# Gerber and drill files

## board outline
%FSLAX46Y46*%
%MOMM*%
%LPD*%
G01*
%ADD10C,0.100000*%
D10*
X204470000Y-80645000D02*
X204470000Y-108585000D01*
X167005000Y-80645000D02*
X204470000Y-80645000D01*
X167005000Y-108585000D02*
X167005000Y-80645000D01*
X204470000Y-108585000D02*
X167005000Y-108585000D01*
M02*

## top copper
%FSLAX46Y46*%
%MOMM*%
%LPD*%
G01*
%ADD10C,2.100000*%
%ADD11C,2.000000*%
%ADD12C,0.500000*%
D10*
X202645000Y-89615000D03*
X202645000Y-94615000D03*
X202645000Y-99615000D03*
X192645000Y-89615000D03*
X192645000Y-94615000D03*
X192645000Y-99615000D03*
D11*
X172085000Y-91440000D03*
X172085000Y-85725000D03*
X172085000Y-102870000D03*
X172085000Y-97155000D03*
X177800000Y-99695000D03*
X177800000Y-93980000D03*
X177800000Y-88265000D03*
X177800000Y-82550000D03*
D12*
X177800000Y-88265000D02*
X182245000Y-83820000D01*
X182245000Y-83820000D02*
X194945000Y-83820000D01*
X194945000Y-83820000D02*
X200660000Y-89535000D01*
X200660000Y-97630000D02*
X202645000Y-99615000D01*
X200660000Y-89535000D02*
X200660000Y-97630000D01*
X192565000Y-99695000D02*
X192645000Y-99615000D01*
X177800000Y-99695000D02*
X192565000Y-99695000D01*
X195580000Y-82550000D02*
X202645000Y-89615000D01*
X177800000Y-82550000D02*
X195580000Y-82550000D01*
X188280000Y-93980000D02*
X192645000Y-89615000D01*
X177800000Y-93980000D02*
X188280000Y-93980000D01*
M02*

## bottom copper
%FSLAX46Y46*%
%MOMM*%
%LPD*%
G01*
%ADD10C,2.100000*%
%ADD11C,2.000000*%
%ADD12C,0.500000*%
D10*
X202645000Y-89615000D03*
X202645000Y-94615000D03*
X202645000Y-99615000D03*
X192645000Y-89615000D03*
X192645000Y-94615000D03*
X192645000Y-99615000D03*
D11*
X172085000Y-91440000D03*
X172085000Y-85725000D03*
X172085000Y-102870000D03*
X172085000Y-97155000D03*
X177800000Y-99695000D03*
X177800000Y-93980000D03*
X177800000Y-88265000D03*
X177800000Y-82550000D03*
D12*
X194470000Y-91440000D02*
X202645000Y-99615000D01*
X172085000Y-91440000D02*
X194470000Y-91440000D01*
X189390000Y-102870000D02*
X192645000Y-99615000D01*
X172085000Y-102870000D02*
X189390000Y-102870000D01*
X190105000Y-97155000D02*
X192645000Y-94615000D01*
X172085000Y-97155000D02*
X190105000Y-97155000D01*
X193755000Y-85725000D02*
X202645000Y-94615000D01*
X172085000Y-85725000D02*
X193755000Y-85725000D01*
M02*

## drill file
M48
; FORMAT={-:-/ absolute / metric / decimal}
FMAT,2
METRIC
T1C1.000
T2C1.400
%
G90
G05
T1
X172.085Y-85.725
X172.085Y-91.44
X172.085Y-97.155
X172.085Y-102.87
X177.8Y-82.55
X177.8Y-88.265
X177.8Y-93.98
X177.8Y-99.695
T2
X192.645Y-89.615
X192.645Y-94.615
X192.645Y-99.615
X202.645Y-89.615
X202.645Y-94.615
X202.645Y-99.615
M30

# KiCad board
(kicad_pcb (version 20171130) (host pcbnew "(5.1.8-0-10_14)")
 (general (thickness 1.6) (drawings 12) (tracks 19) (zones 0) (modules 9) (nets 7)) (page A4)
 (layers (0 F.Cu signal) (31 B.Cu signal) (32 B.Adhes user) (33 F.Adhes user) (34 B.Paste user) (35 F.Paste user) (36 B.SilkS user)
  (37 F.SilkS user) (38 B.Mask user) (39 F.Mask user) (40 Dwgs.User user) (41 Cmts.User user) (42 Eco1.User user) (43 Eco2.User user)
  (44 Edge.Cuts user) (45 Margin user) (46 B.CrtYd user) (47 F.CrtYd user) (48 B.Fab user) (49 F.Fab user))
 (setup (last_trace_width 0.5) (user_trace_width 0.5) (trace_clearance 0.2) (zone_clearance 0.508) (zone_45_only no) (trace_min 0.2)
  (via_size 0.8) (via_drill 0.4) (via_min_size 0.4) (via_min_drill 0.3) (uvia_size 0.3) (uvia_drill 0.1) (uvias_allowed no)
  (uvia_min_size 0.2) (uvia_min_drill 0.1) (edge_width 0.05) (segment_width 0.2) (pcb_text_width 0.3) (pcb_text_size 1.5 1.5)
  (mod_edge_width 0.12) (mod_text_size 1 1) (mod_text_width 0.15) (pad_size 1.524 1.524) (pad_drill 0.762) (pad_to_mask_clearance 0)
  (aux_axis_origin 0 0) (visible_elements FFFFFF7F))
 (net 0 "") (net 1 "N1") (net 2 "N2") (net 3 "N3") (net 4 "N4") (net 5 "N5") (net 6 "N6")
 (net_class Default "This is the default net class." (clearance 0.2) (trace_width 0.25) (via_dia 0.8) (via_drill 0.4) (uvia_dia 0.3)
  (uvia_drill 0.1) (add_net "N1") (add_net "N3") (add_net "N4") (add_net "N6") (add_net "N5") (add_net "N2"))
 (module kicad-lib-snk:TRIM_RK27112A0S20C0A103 (layer F.Cu) (at 207.645 94.615)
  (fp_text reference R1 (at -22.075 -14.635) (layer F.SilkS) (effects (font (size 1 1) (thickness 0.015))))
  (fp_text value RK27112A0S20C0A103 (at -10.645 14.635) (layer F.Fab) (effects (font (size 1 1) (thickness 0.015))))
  (pad 3_1 thru_hole circle (at -5 -5) (size 2.1 2.1) (drill 1.4) (layers *.Cu *.Mask) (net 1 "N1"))
  (pad 2_1 thru_hole circle (at -5 0) (size 2.1 2.1) (drill 1.4) (layers *.Cu *.Mask) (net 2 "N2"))
  (pad 1_1 thru_hole circle (at -5 5) (size 2.1 2.1) (drill 1.4) (layers *.Cu *.Mask) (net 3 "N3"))
  (pad 3_2 thru_hole circle (at -15 -5) (size 2.1 2.1) (drill 1.4) (layers *.Cu *.Mask) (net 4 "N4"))
  (pad 2_2 thru_hole circle (at -15 0) (size 2.1 2.1) (drill 1.4) (layers *.Cu *.Mask) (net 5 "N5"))
  (pad 1_2 thru_hole circle (at -15 5) (size 2.1 2.1) (drill 1.4) (layers *.Cu *.Mask) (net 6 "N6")))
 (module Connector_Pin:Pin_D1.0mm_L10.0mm (layer F.Cu) (at 172.085 91.44)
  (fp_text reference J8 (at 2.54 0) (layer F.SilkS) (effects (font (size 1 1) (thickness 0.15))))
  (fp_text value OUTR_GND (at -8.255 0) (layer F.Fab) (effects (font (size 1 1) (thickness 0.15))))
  (pad 1 thru_hole circle (at 0 0) (size 2 2) (drill 1) (layers *.Cu *.Mask) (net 3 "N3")))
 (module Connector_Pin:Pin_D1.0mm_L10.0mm (layer F.Cu) (at 172.085 85.725)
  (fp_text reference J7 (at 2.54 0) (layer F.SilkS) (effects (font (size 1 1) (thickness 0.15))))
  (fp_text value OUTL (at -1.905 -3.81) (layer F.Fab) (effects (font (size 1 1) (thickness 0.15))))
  (pad 1 thru_hole circle (at 0 0) (size 2 2) (drill 1) (layers *.Cu *.Mask) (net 2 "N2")))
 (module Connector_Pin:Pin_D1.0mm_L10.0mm (layer F.Cu) (at 172.085 102.87)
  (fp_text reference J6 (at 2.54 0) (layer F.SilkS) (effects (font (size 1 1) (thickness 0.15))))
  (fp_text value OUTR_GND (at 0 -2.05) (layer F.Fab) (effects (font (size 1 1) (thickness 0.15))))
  (pad 1 thru_hole circle (at 0 0) (size 2 2) (drill 1) (layers *.Cu *.Mask) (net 6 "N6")))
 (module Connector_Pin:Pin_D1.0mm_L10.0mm (layer F.Cu) (at 172.085 97.155)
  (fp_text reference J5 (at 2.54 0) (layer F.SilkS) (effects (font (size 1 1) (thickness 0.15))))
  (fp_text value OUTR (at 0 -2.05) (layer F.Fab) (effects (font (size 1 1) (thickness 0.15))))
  (pad 1 thru_hole circle (at 0 0) (size 2 2) (drill 1) (layers *.Cu *.Mask) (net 5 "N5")))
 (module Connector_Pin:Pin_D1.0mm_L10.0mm (layer F.Cu) (at 177.8 99.695)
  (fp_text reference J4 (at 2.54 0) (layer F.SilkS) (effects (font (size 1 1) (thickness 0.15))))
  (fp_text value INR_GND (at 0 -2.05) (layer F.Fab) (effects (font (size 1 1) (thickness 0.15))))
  (pad 1 thru_hole circle (at 0 0) (size 2 2) (drill 1) (layers *.Cu *.Mask) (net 6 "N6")))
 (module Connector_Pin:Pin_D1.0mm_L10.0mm (layer F.Cu) (at 177.8 93.98)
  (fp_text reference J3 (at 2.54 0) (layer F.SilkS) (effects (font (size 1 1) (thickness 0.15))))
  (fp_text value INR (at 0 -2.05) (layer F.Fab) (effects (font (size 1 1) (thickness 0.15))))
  (pad 1 thru_hole circle (at 0 0) (size 2 2) (drill 1) (layers *.Cu *.Mask) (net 4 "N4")))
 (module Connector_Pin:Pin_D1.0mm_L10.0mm (layer F.Cu) (at 177.8 88.265)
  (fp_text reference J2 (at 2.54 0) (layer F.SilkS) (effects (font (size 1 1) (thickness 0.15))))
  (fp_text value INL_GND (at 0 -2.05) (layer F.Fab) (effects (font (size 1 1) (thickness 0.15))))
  (pad 1 thru_hole circle (at 0 0) (size 2 2) (drill 1) (layers *.Cu *.Mask) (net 3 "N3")))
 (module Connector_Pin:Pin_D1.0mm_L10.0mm (layer F.Cu) (at 177.8 82.55)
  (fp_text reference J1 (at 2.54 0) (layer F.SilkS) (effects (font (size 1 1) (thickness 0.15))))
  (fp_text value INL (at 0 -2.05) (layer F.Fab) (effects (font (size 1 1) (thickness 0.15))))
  (pad 1 thru_hole circle (at 0 0) (size 2 2) (drill 1) (layers *.Cu *.Mask) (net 1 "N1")))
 (gr_line (start 204.47 80.645) (end 204.47 108.585) (layer Edge.Cuts) (width 0.1))
 (gr_line (start 167.005 80.645) (end 204.47 80.645) (layer Edge.Cuts) (width 0.1))
 (gr_line (start 167.005 108.585) (end 167.005 80.645) (layer Edge.Cuts) (width 0.1))
 (gr_line (start 204.47 108.585) (end 167.005 108.585) (layer Edge.Cuts) (width 0.1))
 (segment (start 177.8 88.265) (end 182.245 83.82) (width 0.5) (layer F.Cu) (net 3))
 (segment (start 182.245 83.82) (end 194.945 83.82) (width 0.5) (layer F.Cu) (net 3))
 (segment (start 194.945 83.82) (end 200.66 89.535) (width 0.5) (layer F.Cu) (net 3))
 (segment (start 200.66 97.63) (end 202.645 99.615) (width 0.5) (layer F.Cu) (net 3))
 (segment (start 200.66 89.535) (end 200.66 97.63) (width 0.5) (layer F.Cu) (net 3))
 (segment (start 194.47 91.44) (end 202.645 99.615) (width 0.5) (layer B.Cu) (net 3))
 (segment (start 172.085 91.44) (end 194.47 91.44) (width 0.5) (layer B.Cu) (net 3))
 (segment (start 192.565 99.695) (end 192.645 99.615) (width 0.5) (layer F.Cu) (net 6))
 (segment (start 177.8 99.695) (end 192.565 99.695) (width 0.5) (layer F.Cu) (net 6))
 (segment (start 189.39 102.87) (end 192.645 99.615) (width 0.5) (layer B.Cu) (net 6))
 (segment (start 172.085 102.87) (end 189.39 102.87) (width 0.5) (layer B.Cu) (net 6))
 (segment (start 195.58 82.55) (end 202.645 89.615) (width 0.5) (layer F.Cu) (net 1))
 (segment (start 177.8 82.55) (end 195.58 82.55) (width 0.5) (layer F.Cu) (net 1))
 (segment (start 188.28 93.98) (end 192.645 89.615) (width 0.5) (layer F.Cu) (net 4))
 (segment (start 177.8 93.98) (end 188.28 93.98) (width 0.5) (layer F.Cu) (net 4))
 (segment (start 190.105 97.155) (end 192.645 94.615) (width 0.5) (layer B.Cu) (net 5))
 (segment (start 172.085 97.155) (end 190.105 97.155) (width 0.5) (layer B.Cu) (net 5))
 (segment (start 193.755 85.725) (end 202.645 94.615) (width 0.5) (layer B.Cu) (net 2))
 (segment (start 172.085 85.725) (end 193.755 85.725) (width 0.5) (layer B.Cu) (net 2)))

